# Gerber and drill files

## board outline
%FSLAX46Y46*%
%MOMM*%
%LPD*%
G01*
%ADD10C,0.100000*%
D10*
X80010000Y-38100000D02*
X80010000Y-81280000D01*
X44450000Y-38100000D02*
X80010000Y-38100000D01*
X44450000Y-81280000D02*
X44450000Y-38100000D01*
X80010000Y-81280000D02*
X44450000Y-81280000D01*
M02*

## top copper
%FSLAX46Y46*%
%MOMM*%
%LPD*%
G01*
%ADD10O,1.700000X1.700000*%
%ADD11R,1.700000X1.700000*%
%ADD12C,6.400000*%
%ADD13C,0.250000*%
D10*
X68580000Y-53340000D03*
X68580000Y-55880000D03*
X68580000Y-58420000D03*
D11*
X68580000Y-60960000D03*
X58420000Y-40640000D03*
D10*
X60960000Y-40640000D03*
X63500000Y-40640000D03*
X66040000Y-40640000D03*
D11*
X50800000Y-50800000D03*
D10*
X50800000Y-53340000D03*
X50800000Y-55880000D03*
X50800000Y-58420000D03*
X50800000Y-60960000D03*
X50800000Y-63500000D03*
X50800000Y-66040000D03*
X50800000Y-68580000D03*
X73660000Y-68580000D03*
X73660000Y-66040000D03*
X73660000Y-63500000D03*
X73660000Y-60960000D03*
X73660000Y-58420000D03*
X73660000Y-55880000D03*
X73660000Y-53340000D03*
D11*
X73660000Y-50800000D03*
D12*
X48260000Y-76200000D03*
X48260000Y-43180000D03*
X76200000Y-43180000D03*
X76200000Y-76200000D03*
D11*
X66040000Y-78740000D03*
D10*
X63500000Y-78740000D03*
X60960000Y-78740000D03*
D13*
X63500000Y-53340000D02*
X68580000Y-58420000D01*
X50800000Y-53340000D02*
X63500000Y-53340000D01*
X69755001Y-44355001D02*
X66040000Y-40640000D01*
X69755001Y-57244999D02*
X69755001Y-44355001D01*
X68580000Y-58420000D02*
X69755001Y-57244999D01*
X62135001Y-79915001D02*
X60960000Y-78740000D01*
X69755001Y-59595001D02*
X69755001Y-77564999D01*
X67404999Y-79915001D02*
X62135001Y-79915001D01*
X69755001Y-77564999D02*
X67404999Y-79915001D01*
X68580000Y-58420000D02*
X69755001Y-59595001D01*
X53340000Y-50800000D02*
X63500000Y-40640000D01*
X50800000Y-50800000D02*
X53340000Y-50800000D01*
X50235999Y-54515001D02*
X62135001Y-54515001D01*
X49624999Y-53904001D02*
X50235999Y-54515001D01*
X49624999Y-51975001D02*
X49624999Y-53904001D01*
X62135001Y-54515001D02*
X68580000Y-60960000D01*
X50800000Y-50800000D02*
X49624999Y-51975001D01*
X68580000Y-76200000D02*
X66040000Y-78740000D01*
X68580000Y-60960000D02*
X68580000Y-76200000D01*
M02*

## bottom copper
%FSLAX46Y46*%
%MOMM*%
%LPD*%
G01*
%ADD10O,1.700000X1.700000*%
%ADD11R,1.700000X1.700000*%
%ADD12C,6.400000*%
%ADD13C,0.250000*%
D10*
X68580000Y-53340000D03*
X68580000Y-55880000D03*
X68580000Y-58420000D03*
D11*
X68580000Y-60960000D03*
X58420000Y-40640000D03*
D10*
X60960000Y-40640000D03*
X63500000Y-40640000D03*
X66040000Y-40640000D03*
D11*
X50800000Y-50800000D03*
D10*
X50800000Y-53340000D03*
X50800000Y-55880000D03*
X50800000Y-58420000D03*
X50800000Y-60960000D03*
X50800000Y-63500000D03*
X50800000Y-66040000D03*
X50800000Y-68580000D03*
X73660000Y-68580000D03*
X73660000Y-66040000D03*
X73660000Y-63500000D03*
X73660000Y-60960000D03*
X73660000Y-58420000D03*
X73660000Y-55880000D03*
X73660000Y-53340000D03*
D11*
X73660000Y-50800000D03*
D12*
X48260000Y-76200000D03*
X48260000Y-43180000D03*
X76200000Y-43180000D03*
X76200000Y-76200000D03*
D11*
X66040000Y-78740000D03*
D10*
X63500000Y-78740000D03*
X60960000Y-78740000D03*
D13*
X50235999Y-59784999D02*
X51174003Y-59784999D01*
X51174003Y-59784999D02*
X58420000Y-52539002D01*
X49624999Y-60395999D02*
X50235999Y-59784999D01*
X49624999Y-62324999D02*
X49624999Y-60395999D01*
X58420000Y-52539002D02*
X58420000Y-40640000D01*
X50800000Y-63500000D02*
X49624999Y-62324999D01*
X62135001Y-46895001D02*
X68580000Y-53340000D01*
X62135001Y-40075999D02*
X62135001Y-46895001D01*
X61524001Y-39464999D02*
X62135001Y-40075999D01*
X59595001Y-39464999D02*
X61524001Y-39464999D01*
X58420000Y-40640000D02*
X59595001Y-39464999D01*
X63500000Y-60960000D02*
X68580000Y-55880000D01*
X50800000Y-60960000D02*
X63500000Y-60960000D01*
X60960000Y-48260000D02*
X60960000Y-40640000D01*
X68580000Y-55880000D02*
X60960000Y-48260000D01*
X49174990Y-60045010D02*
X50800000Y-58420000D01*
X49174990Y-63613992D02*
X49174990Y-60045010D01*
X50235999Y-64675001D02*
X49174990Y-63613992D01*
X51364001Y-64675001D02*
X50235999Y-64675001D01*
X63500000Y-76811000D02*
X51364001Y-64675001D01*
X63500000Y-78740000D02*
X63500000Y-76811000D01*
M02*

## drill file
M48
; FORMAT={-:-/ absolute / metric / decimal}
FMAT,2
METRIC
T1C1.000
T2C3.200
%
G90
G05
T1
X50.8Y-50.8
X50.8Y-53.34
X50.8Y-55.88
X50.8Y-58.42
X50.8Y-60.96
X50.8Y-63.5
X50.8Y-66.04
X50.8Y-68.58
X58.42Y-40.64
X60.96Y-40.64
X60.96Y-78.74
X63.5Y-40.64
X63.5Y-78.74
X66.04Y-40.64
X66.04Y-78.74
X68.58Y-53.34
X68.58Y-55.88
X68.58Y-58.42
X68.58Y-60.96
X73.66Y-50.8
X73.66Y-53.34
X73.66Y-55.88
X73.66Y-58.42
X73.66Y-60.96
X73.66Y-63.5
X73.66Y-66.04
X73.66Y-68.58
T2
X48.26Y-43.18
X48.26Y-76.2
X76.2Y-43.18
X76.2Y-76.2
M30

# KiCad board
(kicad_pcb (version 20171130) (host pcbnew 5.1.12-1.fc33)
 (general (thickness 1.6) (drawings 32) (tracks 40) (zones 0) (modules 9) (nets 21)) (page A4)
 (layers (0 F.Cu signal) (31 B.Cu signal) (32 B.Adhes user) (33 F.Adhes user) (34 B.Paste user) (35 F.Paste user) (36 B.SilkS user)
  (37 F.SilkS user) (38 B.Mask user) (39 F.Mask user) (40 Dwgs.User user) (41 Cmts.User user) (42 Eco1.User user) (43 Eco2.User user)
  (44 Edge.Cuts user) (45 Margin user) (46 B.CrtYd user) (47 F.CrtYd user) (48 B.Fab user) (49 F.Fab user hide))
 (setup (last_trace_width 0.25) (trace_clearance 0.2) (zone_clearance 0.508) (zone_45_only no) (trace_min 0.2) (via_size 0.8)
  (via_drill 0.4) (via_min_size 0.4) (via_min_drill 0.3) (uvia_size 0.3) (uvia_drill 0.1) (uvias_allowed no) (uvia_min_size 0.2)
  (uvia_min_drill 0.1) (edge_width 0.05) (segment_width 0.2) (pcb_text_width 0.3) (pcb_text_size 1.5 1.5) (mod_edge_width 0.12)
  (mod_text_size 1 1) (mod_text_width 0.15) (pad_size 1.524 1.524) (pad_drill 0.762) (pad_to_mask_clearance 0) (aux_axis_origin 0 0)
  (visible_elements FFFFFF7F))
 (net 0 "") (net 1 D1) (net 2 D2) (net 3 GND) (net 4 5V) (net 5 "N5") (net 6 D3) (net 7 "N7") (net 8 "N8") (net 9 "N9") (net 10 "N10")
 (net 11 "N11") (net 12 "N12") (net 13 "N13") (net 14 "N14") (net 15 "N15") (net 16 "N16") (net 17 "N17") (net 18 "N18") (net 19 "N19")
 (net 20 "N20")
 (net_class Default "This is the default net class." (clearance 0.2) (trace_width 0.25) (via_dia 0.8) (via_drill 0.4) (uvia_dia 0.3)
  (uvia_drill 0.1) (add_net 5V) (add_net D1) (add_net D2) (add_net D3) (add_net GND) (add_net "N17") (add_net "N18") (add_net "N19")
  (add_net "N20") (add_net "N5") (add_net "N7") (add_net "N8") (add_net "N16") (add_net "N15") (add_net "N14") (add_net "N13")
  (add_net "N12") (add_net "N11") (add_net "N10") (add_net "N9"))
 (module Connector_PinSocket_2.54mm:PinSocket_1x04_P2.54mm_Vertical (layer B.Cu) (at 68.58 60.96)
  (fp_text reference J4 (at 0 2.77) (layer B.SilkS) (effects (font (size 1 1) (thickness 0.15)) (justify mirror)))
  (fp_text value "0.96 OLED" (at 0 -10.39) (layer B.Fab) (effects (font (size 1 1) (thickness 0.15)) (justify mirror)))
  (pad 4 thru_hole oval (at 0 -7.62) (size 1.7 1.7) (drill 1) (layers *.Cu *.Mask) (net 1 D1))
  (pad 3 thru_hole oval (at 0 -5.08) (size 1.7 1.7) (drill 1) (layers *.Cu *.Mask) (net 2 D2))
  (pad 2 thru_hole oval (at 0 -2.54) (size 1.7 1.7) (drill 1) (layers *.Cu *.Mask) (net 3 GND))
  (pad 1 thru_hole rect (at 0 0) (size 1.7 1.7) (drill 1) (layers *.Cu *.Mask) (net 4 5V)))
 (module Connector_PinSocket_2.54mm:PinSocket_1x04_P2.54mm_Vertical (layer B.Cu) (at 58.42 40.64 270)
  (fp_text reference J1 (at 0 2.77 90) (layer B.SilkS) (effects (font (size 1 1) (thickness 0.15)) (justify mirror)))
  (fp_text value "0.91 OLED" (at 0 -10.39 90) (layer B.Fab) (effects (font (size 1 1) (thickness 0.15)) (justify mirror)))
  (pad 1 thru_hole rect (at 0 0 270) (size 1.7 1.7) (drill 1) (layers *.Cu *.Mask) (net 1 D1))
  (pad 2 thru_hole oval (at 0 -2.54 270) (size 1.7 1.7) (drill 1) (layers *.Cu *.Mask) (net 2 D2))
  (pad 3 thru_hole oval (at 0 -5.08 270) (size 1.7 1.7) (drill 1) (layers *.Cu *.Mask) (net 4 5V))
  (pad 4 thru_hole oval (at 0 -7.62 270) (size 1.7 1.7) (drill 1) (layers *.Cu *.Mask) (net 3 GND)))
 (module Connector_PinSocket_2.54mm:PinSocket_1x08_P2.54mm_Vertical (layer F.Cu) (at 50.8 50.8)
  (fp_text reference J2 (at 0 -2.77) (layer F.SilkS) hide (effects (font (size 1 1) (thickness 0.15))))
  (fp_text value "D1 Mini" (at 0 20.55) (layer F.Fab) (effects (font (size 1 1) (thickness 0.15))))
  (pad 1 thru_hole rect (at 0 0) (size 1.7 1.7) (drill 1) (layers *.Cu *.Mask) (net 4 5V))
  (pad 2 thru_hole oval (at 0 2.54) (size 1.7 1.7) (drill 1) (layers *.Cu *.Mask) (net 3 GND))
  (pad 3 thru_hole oval (at 0 5.08) (size 1.7 1.7) (drill 1) (layers *.Cu *.Mask) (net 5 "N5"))
  (pad 4 thru_hole oval (at 0 7.62) (size 1.7 1.7) (drill 1) (layers *.Cu *.Mask) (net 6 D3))
  (pad 5 thru_hole oval (at 0 10.16) (size 1.7 1.7) (drill 1) (layers *.Cu *.Mask) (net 2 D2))
  (pad 6 thru_hole oval (at 0 12.7) (size 1.7 1.7) (drill 1) (layers *.Cu *.Mask) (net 1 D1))
  (pad 7 thru_hole oval (at 0 15.24) (size 1.7 1.7) (drill 1) (layers *.Cu *.Mask) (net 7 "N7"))
  (pad 8 thru_hole oval (at 0 17.78) (size 1.7 1.7) (drill 1) (layers *.Cu *.Mask) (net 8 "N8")))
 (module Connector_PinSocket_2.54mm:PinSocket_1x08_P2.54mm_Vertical (layer F.Cu) (at 73.66 50.8)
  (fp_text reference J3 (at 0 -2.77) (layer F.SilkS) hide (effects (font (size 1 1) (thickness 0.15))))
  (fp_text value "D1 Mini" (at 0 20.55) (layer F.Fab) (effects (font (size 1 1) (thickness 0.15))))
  (pad 8 thru_hole oval (at 0 17.78) (size 1.7 1.7) (drill 1) (layers *.Cu *.Mask) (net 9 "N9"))
  (pad 7 thru_hole oval (at 0 15.24) (size 1.7 1.7) (drill 1) (layers *.Cu *.Mask) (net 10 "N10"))
  (pad 6 thru_hole oval (at 0 12.7) (size 1.7 1.7) (drill 1) (layers *.Cu *.Mask) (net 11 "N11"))
  (pad 5 thru_hole oval (at 0 10.16) (size 1.7 1.7) (drill 1) (layers *.Cu *.Mask) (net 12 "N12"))
  (pad 4 thru_hole oval (at 0 7.62) (size 1.7 1.7) (drill 1) (layers *.Cu *.Mask) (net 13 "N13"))
  (pad 3 thru_hole oval (at 0 5.08) (size 1.7 1.7) (drill 1) (layers *.Cu *.Mask) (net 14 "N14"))
  (pad 2 thru_hole oval (at 0 2.54) (size 1.7 1.7) (drill 1) (layers *.Cu *.Mask) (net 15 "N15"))
  (pad 1 thru_hole rect (at 0 0) (size 1.7 1.7) (drill 1) (layers *.Cu *.Mask) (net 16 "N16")))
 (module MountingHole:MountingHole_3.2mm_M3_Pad (layer F.Cu) (at 48.26 76.2)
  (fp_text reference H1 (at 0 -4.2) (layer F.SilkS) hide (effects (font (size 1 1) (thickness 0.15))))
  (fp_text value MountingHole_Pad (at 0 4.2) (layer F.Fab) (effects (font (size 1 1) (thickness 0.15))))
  (pad 1 thru_hole circle (at 0 0) (size 6.4 6.4) (drill 3.2) (layers *.Cu *.Mask) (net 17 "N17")))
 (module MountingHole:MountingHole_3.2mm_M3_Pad (layer F.Cu) (at 48.26 43.18)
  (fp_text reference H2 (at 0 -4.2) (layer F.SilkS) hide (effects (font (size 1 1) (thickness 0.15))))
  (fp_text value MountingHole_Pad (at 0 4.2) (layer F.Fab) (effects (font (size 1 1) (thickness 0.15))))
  (pad 1 thru_hole circle (at 0 0) (size 6.4 6.4) (drill 3.2) (layers *.Cu *.Mask) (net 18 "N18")))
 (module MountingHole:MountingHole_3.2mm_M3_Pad (layer F.Cu) (at 76.2 43.18)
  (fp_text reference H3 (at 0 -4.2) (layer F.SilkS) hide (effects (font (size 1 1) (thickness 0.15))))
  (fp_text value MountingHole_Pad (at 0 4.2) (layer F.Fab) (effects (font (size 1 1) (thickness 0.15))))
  (pad 1 thru_hole circle (at 0 0) (size 6.4 6.4) (drill 3.2) (layers *.Cu *.Mask) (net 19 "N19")))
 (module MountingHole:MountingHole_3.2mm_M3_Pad (layer F.Cu) (at 76.2 76.2)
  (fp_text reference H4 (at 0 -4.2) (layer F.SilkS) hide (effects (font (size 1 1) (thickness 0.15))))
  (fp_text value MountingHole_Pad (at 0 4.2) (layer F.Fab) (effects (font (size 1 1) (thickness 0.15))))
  (pad 1 thru_hole circle (at 0 0) (size 6.4 6.4) (drill 3.2) (layers *.Cu *.Mask) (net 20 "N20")))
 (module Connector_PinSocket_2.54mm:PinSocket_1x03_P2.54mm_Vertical (layer F.Cu) (at 66.04 78.74 270)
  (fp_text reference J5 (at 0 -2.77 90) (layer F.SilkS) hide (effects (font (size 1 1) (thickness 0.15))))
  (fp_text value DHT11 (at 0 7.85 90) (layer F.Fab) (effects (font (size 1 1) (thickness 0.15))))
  (pad 1 thru_hole rect (at 0 0 270) (size 1.7 1.7) (drill 1) (layers *.Cu *.Mask) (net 4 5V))
  (pad 2 thru_hole oval (at 0 2.54 270) (size 1.7 1.7) (drill 1) (layers *.Cu *.Mask) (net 6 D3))
  (pad 3 thru_hole oval (at 0 5.08 270) (size 1.7 1.7) (drill 1) (layers *.Cu *.Mask) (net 3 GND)))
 (gr_line (start 80.01 38.1) (end 80.01 81.28) (layer Edge.Cuts) (width 0.1))
 (gr_line (start 44.45 38.1) (end 80.01 38.1) (layer Edge.Cuts) (width 0.1))
 (gr_line (start 44.45 81.28) (end 44.45 38.1) (layer Edge.Cuts) (width 0.1))
 (gr_line (start 80.01 81.28) (end 44.45 81.28) (layer Edge.Cuts) (width 0.1))
 (segment (start 63.5 53.34) (end 68.58 58.42) (width 0.25) (layer F.Cu) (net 3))
 (segment (start 50.8 53.34) (end 63.5 53.34) (width 0.25) (layer F.Cu) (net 3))
 (segment (start 69.755001 44.355001) (end 66.04 40.64) (width 0.25) (layer F.Cu) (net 3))
 (segment (start 69.755001 57.244999) (end 69.755001 44.355001) (width 0.25) (layer F.Cu) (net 3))
 (segment (start 68.58 58.42) (end 69.755001 57.244999) (width 0.25) (layer F.Cu) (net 3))
 (segment (start 62.135001 79.915001) (end 60.96 78.74) (width 0.25) (layer F.Cu) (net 3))
 (segment (start 69.755001 59.595001) (end 69.755001 77.564999) (width 0.25) (layer F.Cu) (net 3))
 (segment (start 67.404999 79.915001) (end 62.135001 79.915001) (width 0.25) (layer F.Cu) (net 3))
 (segment (start 69.755001 77.564999) (end 67.404999 79.915001) (width 0.25) (layer F.Cu) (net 3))
 (segment (start 68.58 58.42) (end 69.755001 59.595001) (width 0.25) (layer F.Cu) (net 3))
 (segment (start 50.235999 59.784999) (end 51.174003 59.784999) (width 0.25) (layer B.Cu) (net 1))
 (segment (start 51.174003 59.784999) (end 58.42 52.539002) (width 0.25) (layer B.Cu) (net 1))
 (segment (start 49.624999 60.395999) (end 50.235999 59.784999) (width 0.25) (layer B.Cu) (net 1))
 (segment (start 49.624999 62.324999) (end 49.624999 60.395999) (width 0.25) (layer B.Cu) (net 1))
 (segment (start 58.42 52.539002) (end 58.42 40.64) (width 0.25) (layer B.Cu) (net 1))
 (segment (start 50.8 63.5) (end 49.624999 62.324999) (width 0.25) (layer B.Cu) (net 1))
 (segment (start 62.135001 46.895001) (end 68.58 53.34) (width 0.25) (layer B.Cu) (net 1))
 (segment (start 62.135001 40.075999) (end 62.135001 46.895001) (width 0.25) (layer B.Cu) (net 1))
 (segment (start 61.524001 39.464999) (end 62.135001 40.075999) (width 0.25) (layer B.Cu) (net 1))
 (segment (start 59.595001 39.464999) (end 61.524001 39.464999) (width 0.25) (layer B.Cu) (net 1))
 (segment (start 58.42 40.64) (end 59.595001 39.464999) (width 0.25) (layer B.Cu) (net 1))
 (segment (start 63.5 60.96) (end 68.58 55.88) (width 0.25) (layer B.Cu) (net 2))
 (segment (start 50.8 60.96) (end 63.5 60.96) (width 0.25) (layer B.Cu) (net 2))
 (segment (start 60.96 48.26) (end 60.96 40.64) (width 0.25) (layer B.Cu) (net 2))
 (segment (start 68.58 55.88) (end 60.96 48.26) (width 0.25) (layer B.Cu) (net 2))
 (segment (start 53.34 50.8) (end 63.5 40.64) (width 0.25) (layer F.Cu) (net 4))
 (segment (start 50.8 50.8) (end 53.34 50.8) (width 0.25) (layer F.Cu) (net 4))
 (segment (start 50.235999 54.515001) (end 62.135001 54.515001) (width 0.25) (layer F.Cu) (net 4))
 (segment (start 49.624999 53.904001) (end 50.235999 54.515001) (width 0.25) (layer F.Cu) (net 4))
 (segment (start 49.624999 51.975001) (end 49.624999 53.904001) (width 0.25) (layer F.Cu) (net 4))
 (segment (start 62.135001 54.515001) (end 68.58 60.96) (width 0.25) (layer F.Cu) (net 4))
 (segment (start 50.8 50.8) (end 49.624999 51.975001) (width 0.25) (layer F.Cu) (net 4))
 (segment (start 68.58 76.2) (end 66.04 78.74) (width 0.25) (layer F.Cu) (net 4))
 (segment (start 68.58 60.96) (end 68.58 76.2) (width 0.25) (layer F.Cu) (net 4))
 (segment (start 49.17499 60.04501) (end 50.8 58.42) (width 0.25) (layer B.Cu) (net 6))
 (segment (start 49.17499 63.613992) (end 49.17499 60.04501) (width 0.25) (layer B.Cu) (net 6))
 (segment (start 50.235999 64.675001) (end 49.17499 63.613992) (width 0.25) (layer B.Cu) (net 6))
 (segment (start 51.364001 64.675001) (end 50.235999 64.675001) (width 0.25) (layer B.Cu) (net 6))
 (segment (start 63.5 76.811) (end 51.364001 64.675001) (width 0.25) (layer B.Cu) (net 6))
 (segment (start 63.5 78.74) (end 63.5 76.811) (width 0.25) (layer B.Cu) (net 6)))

